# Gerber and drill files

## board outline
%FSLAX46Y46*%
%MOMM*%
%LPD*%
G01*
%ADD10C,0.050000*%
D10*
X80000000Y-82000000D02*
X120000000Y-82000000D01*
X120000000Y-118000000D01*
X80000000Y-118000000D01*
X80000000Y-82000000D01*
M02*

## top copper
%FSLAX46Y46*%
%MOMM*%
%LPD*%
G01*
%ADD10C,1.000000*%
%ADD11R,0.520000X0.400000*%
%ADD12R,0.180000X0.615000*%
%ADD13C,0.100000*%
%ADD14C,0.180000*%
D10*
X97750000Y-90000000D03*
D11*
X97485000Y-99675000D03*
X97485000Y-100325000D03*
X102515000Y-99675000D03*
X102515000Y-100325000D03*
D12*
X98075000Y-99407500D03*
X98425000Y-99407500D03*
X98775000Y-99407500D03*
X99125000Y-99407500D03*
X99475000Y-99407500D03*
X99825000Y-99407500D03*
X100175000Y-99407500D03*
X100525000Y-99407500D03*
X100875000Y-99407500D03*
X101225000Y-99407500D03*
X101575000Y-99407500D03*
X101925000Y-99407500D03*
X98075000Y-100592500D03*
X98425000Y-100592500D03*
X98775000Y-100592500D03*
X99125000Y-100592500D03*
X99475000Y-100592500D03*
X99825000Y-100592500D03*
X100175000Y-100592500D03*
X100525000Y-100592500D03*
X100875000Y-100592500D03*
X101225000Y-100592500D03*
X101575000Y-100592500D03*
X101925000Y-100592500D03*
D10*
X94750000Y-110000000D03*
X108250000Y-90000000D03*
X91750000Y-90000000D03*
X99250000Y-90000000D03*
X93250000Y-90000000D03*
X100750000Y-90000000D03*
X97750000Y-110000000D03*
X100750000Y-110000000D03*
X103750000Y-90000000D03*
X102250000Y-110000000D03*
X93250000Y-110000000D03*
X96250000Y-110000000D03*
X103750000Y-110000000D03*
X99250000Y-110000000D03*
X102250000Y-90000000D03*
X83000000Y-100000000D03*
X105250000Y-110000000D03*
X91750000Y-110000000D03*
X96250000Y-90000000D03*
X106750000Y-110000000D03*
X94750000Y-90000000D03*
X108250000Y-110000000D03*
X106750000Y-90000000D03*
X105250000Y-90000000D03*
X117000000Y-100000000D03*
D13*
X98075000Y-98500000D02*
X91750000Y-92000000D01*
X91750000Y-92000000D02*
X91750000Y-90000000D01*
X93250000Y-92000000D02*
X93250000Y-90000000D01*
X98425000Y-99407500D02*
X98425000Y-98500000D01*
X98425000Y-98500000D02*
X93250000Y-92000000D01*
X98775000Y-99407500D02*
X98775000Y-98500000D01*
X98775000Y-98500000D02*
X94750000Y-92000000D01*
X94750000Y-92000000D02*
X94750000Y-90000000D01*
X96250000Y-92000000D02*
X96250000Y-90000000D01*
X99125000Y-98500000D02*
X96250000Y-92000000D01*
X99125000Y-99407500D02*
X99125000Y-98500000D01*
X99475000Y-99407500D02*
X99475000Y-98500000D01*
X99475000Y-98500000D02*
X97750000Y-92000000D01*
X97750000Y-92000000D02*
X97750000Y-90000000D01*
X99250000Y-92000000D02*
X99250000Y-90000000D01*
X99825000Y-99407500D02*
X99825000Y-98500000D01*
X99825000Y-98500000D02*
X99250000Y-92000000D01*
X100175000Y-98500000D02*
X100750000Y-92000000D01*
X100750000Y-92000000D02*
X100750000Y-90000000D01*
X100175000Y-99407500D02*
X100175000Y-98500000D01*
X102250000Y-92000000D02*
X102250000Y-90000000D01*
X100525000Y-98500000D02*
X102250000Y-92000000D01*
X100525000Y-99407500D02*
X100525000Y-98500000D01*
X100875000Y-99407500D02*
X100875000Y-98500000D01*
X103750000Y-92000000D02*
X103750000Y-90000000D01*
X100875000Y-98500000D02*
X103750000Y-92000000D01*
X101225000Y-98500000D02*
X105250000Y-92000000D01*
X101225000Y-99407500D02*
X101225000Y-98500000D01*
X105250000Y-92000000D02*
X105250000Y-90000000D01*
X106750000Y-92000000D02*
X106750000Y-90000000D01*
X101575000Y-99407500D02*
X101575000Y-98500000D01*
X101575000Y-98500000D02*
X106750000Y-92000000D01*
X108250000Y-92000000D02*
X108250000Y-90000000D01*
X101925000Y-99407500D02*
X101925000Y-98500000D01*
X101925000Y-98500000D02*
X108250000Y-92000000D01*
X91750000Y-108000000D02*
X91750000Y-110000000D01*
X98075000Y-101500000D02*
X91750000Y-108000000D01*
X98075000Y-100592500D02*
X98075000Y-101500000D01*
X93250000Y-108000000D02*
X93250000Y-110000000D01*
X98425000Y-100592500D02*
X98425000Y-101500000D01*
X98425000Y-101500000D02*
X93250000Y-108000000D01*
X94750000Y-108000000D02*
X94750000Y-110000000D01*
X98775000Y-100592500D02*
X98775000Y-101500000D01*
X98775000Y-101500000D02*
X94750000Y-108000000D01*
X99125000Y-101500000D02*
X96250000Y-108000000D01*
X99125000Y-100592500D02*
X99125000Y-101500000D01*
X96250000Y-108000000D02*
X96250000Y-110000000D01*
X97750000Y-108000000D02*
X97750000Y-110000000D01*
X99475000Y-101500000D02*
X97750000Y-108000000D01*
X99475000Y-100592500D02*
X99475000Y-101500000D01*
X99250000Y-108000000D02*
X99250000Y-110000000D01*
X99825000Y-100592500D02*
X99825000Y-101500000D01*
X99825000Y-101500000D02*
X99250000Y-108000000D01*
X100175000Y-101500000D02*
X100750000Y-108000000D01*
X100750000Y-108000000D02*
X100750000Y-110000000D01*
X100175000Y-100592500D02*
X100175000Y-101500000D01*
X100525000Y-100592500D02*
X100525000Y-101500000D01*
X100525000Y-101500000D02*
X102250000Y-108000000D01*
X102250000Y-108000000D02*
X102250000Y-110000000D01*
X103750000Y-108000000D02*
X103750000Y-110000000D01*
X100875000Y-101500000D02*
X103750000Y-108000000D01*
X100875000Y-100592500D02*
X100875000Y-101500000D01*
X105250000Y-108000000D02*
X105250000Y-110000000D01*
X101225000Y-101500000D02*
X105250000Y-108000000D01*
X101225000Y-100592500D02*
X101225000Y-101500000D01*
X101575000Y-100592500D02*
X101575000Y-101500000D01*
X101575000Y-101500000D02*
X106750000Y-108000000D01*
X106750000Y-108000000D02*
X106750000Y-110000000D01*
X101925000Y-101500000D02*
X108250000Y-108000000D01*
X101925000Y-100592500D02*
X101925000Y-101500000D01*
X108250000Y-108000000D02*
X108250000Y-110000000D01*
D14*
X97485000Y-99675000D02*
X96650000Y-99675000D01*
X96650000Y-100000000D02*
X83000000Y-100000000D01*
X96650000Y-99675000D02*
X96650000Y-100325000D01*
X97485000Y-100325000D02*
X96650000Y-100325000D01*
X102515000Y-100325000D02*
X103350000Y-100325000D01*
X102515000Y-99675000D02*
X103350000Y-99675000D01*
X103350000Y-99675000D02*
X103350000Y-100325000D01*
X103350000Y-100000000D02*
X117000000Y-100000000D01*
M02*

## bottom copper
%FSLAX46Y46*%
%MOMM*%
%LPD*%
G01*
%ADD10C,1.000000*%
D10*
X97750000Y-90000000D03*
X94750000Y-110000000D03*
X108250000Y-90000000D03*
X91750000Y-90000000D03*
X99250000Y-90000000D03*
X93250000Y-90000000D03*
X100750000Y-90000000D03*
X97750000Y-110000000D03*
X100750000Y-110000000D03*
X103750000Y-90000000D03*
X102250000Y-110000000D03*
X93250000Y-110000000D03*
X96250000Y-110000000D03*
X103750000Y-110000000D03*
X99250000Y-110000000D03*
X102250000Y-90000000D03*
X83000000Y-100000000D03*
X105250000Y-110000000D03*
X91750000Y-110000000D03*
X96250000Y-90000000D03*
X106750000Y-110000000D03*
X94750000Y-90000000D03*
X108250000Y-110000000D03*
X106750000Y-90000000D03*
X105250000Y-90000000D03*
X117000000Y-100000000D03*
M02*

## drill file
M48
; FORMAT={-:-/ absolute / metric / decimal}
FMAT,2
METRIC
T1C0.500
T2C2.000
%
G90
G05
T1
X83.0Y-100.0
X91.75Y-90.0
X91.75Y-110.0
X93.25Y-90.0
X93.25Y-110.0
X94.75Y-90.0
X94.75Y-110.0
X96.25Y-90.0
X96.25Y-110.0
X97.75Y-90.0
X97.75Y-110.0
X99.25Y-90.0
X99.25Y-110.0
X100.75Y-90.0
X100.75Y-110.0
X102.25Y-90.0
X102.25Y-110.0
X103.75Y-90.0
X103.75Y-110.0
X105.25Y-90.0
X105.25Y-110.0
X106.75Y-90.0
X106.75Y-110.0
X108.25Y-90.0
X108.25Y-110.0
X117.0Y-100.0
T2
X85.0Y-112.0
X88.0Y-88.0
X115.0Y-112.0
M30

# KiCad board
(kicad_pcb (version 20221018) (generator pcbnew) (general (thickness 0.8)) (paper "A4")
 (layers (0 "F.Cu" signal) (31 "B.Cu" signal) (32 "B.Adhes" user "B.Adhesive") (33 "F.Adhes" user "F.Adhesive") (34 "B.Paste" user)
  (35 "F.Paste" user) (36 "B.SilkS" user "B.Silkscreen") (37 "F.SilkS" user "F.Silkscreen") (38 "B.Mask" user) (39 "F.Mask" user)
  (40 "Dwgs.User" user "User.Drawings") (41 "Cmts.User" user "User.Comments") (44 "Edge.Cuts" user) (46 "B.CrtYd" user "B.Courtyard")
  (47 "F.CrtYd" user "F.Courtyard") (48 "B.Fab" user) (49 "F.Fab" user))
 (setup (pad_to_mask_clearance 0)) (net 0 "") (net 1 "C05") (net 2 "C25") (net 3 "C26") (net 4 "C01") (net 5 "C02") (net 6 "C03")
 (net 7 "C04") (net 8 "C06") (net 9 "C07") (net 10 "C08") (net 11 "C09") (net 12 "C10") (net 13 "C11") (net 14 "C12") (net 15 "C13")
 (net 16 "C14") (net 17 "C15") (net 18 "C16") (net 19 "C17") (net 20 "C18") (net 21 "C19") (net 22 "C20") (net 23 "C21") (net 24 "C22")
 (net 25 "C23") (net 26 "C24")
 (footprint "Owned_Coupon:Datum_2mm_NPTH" (layer "F.Cu") (at 85 112)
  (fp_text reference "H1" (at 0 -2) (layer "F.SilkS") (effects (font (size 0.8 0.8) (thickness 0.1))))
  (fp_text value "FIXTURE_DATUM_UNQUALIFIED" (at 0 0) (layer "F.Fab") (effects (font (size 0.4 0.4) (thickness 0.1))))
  (pad "" np_thru_hole circle (at 0 0) (size 2 2) (drill 2) (layers "*.Cu" "*.Mask")))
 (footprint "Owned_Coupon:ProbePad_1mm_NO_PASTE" (layer "F.Cu") (at 97.75 90)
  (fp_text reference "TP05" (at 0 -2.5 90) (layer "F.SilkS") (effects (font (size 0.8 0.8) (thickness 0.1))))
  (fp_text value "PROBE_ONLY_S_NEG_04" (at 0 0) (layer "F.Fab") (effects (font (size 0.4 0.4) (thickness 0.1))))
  (pad "1" thru_hole circle (at 0 0) (size 1 1) (drill 0.5) (layers "*.Cu" "*.Mask") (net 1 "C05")))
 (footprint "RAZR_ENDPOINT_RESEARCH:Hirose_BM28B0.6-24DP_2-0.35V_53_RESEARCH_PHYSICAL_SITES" (layer "F.Cu") (at 100 100)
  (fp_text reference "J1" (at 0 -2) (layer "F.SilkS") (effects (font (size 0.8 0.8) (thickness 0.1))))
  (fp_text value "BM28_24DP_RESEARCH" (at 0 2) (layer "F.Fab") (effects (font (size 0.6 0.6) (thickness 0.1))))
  (pad "P_L" smd rect (at -2.515 -0.325) (size 0.52 0.4) (layers "F.Cu" "F.Mask") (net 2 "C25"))
  (pad "P_L" smd rect (at -2.515 0.325) (size 0.52 0.4) (layers "F.Cu" "F.Mask") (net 2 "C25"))
  (pad "P_R" smd rect (at 2.515 -0.325) (size 0.52 0.4) (layers "F.Cu" "F.Mask") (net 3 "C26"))
  (pad "P_R" smd rect (at 2.515 0.325) (size 0.52 0.4) (layers "F.Cu" "F.Mask") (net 3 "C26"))
  (pad "S_NEG_00" smd rect (at -1.925 -0.5925) (size 0.18 0.615) (layers "F.Cu" "F.Mask") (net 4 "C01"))
  (pad "S_NEG_01" smd rect (at -1.575 -0.5925) (size 0.18 0.615) (layers "F.Cu" "F.Mask") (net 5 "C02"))
  (pad "S_NEG_02" smd rect (at -1.225 -0.5925) (size 0.18 0.615) (layers "F.Cu" "F.Mask") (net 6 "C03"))
  (pad "S_NEG_03" smd rect (at -0.875 -0.5925) (size 0.18 0.615) (layers "F.Cu" "F.Mask") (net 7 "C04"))
  (pad "S_NEG_04" smd rect (at -0.525 -0.5925) (size 0.18 0.615) (layers "F.Cu" "F.Mask") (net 1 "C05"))
  (pad "S_NEG_05" smd rect (at -0.175 -0.5925) (size 0.18 0.615) (layers "F.Cu" "F.Mask") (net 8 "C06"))
  (pad "S_NEG_06" smd rect (at 0.175 -0.5925) (size 0.18 0.615) (layers "F.Cu" "F.Mask") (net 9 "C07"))
  (pad "S_NEG_07" smd rect (at 0.525 -0.5925) (size 0.18 0.615) (layers "F.Cu" "F.Mask") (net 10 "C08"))
  (pad "S_NEG_08" smd rect (at 0.875 -0.5925) (size 0.18 0.615) (layers "F.Cu" "F.Mask") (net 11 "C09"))
  (pad "S_NEG_09" smd rect (at 1.225 -0.5925) (size 0.18 0.615) (layers "F.Cu" "F.Mask") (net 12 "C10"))
  (pad "S_NEG_10" smd rect (at 1.575 -0.5925) (size 0.18 0.615) (layers "F.Cu" "F.Mask") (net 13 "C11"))
  (pad "S_NEG_11" smd rect (at 1.925 -0.5925) (size 0.18 0.615) (layers "F.Cu" "F.Mask") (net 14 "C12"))
  (pad "S_POS_00" smd rect (at -1.925 0.5925) (size 0.18 0.615) (layers "F.Cu" "F.Mask") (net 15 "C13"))
  (pad "S_POS_01" smd rect (at -1.575 0.5925) (size 0.18 0.615) (layers "F.Cu" "F.Mask") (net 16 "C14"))
  (pad "S_POS_02" smd rect (at -1.225 0.5925) (size 0.18 0.615) (layers "F.Cu" "F.Mask") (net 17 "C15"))
  (pad "S_POS_03" smd rect (at -0.875 0.5925) (size 0.18 0.615) (layers "F.Cu" "F.Mask") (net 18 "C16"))
  (pad "S_POS_04" smd rect (at -0.525 0.5925) (size 0.18 0.615) (layers "F.Cu" "F.Mask") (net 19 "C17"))
  (pad "S_POS_05" smd rect (at -0.175 0.5925) (size 0.18 0.615) (layers "F.Cu" "F.Mask") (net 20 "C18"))
  (pad "S_POS_06" smd rect (at 0.175 0.5925) (size 0.18 0.615) (layers "F.Cu" "F.Mask") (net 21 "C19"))
  (pad "S_POS_07" smd rect (at 0.525 0.5925) (size 0.18 0.615) (layers "F.Cu" "F.Mask") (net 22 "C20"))
  (pad "S_POS_08" smd rect (at 0.875 0.5925) (size 0.18 0.615) (layers "F.Cu" "F.Mask") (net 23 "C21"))
  (pad "S_POS_09" smd rect (at 1.225 0.5925) (size 0.18 0.615) (layers "F.Cu" "F.Mask") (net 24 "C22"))
  (pad "S_POS_10" smd rect (at 1.575 0.5925) (size 0.18 0.615) (layers "F.Cu" "F.Mask") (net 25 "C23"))
  (pad "S_POS_11" smd rect (at 1.925 0.5925) (size 0.18 0.615) (layers "F.Cu" "F.Mask") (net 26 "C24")))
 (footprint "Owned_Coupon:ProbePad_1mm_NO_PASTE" (layer "F.Cu") (at 94.75 110)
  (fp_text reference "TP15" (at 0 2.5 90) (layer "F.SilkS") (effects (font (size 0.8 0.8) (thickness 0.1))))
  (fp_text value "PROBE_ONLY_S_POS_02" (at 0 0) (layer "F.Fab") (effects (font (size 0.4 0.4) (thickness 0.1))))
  (pad "1" thru_hole circle (at 0 0) (size 1 1) (drill 0.5) (layers "*.Cu" "*.Mask") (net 17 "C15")))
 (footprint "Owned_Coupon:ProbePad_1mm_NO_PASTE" (layer "F.Cu") (at 108.25 90)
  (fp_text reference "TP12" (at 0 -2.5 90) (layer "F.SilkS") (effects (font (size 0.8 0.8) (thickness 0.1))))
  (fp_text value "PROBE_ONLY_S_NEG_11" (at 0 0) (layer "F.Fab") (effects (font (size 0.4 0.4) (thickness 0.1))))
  (pad "1" thru_hole circle (at 0 0) (size 1 1) (drill 0.5) (layers "*.Cu" "*.Mask") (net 14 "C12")))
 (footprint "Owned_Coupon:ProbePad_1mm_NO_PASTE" (layer "F.Cu") (at 91.75 90)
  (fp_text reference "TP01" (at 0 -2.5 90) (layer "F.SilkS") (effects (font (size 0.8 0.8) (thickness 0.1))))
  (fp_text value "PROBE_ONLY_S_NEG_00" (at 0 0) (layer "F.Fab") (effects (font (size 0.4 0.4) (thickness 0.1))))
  (pad "1" thru_hole circle (at 0 0) (size 1 1) (drill 0.5) (layers "*.Cu" "*.Mask") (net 4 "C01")))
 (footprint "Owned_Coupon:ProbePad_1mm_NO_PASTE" (layer "F.Cu") (at 99.25 90)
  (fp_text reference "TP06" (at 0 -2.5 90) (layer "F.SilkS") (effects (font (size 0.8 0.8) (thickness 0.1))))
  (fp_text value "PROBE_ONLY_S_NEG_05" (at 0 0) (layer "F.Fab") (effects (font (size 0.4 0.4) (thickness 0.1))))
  (pad "1" thru_hole circle (at 0 0) (size 1 1) (drill 0.5) (layers "*.Cu" "*.Mask") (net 8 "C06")))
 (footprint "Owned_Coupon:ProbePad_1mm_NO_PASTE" (layer "F.Cu") (at 93.25 90)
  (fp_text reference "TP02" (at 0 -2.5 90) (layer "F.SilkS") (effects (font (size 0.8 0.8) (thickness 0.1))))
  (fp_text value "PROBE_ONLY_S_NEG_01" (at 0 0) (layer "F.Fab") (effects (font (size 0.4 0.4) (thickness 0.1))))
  (pad "1" thru_hole circle (at 0 0) (size 1 1) (drill 0.5) (layers "*.Cu" "*.Mask") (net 5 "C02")))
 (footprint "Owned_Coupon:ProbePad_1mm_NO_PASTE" (layer "F.Cu") (at 100.75 90)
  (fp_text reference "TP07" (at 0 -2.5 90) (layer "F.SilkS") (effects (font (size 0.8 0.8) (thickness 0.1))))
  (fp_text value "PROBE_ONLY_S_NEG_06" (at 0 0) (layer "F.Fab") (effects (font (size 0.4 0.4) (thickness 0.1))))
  (pad "1" thru_hole circle (at 0 0) (size 1 1) (drill 0.5) (layers "*.Cu" "*.Mask") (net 9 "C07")))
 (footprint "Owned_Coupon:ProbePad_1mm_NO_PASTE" (layer "F.Cu") (at 97.75 110)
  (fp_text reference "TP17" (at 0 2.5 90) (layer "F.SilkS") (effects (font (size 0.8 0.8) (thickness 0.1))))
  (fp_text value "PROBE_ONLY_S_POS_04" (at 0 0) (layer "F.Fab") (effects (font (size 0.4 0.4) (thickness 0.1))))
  (pad "1" thru_hole circle (at 0 0) (size 1 1) (drill 0.5) (layers "*.Cu" "*.Mask") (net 19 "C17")))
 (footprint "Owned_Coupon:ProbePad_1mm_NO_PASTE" (layer "F.Cu") (at 100.75 110)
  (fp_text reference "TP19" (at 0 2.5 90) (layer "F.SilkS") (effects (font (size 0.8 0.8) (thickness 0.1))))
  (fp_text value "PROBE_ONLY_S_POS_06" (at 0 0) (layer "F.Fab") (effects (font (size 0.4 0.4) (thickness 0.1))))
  (pad "1" thru_hole circle (at 0 0) (size 1 1) (drill 0.5) (layers "*.Cu" "*.Mask") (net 21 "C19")))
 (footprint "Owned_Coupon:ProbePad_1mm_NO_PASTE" (layer "F.Cu") (at 103.75 90)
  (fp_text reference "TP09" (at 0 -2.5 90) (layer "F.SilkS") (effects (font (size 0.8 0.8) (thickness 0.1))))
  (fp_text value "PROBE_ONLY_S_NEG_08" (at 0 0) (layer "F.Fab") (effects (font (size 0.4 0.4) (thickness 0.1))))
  (pad "1" thru_hole circle (at 0 0) (size 1 1) (drill 0.5) (layers "*.Cu" "*.Mask") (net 11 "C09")))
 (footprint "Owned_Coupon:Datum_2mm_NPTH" (layer "F.Cu") (at 115 112)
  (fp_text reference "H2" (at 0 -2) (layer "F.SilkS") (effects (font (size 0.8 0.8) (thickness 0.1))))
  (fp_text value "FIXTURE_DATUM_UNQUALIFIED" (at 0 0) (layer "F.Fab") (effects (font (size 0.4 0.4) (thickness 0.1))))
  (pad "" np_thru_hole circle (at 0 0) (size 2 2) (drill 2) (layers "*.Cu" "*.Mask")))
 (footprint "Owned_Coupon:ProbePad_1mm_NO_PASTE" (layer "F.Cu") (at 102.25 110)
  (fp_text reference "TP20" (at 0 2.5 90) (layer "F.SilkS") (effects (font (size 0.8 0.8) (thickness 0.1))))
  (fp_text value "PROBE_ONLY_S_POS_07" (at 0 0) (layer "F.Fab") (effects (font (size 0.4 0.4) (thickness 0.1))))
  (pad "1" thru_hole circle (at 0 0) (size 1 1) (drill 0.5) (layers "*.Cu" "*.Mask") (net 22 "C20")))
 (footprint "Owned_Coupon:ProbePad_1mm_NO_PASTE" (layer "F.Cu") (at 93.25 110)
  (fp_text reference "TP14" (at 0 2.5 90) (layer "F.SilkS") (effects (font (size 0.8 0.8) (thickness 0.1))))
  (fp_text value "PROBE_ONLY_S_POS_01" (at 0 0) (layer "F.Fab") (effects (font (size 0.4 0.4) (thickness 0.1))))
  (pad "1" thru_hole circle (at 0 0) (size 1 1) (drill 0.5) (layers "*.Cu" "*.Mask") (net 16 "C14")))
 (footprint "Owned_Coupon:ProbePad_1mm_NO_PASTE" (layer "F.Cu") (at 96.25 110)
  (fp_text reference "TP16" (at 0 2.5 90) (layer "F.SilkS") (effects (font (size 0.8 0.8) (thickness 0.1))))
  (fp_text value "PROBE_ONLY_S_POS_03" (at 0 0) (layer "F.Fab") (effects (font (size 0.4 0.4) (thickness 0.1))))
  (pad "1" thru_hole circle (at 0 0) (size 1 1) (drill 0.5) (layers "*.Cu" "*.Mask") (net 18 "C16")))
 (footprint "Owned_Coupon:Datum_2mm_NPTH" (layer "F.Cu") (at 88 88)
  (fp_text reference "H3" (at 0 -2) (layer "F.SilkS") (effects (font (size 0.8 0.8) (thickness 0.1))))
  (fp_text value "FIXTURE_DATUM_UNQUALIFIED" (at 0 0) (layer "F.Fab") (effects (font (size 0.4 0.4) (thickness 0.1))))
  (pad "" np_thru_hole circle (at 0 0) (size 2 2) (drill 2) (layers "*.Cu" "*.Mask")))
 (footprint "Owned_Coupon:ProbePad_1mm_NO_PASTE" (layer "F.Cu") (at 103.75 110)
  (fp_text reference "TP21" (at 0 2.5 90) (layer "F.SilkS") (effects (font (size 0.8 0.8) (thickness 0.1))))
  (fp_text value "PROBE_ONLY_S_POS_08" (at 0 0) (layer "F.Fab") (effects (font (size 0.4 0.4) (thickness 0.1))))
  (pad "1" thru_hole circle (at 0 0) (size 1 1) (drill 0.5) (layers "*.Cu" "*.Mask") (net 23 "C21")))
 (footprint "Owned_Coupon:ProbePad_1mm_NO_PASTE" (layer "F.Cu") (at 99.25 110)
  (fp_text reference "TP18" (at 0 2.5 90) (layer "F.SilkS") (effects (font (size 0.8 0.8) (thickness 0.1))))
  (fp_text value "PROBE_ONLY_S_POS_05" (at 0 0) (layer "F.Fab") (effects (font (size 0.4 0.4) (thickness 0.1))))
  (pad "1" thru_hole circle (at 0 0) (size 1 1) (drill 0.5) (layers "*.Cu" "*.Mask") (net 20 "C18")))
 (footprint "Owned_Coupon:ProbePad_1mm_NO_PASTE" (layer "F.Cu") (at 102.25 90)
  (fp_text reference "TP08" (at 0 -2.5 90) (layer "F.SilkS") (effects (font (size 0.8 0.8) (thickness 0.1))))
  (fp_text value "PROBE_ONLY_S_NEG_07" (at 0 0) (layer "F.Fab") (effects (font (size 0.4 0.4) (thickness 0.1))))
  (pad "1" thru_hole circle (at 0 0) (size 1 1) (drill 0.5) (layers "*.Cu" "*.Mask") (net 10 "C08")))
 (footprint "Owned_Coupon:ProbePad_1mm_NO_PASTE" (layer "F.Cu") (at 83 100)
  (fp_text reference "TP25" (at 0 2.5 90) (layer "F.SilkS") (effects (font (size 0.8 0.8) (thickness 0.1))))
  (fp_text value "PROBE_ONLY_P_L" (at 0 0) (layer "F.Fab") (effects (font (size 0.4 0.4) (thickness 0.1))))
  (pad "1" thru_hole circle (at 0 0) (size 1 1) (drill 0.5) (layers "*.Cu" "*.Mask") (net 2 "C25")))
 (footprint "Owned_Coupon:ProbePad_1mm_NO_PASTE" (layer "F.Cu") (at 105.25 110)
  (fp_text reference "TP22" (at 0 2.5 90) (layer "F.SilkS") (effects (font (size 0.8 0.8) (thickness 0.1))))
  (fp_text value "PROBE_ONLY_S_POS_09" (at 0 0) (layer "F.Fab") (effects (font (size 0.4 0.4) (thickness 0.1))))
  (pad "1" thru_hole circle (at 0 0) (size 1 1) (drill 0.5) (layers "*.Cu" "*.Mask") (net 24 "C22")))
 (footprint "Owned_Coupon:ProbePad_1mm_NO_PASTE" (layer "F.Cu") (at 91.75 110)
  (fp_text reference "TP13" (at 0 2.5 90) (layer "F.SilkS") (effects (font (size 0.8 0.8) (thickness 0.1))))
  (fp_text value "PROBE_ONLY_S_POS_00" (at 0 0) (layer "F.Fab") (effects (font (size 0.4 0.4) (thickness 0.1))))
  (pad "1" thru_hole circle (at 0 0) (size 1 1) (drill 0.5) (layers "*.Cu" "*.Mask") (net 15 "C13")))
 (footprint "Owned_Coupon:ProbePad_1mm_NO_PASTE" (layer "F.Cu") (at 96.25 90)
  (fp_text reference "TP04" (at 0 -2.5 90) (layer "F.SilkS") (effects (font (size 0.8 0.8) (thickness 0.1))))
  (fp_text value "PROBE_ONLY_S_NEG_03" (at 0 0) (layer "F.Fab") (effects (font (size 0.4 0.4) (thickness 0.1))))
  (pad "1" thru_hole circle (at 0 0) (size 1 1) (drill 0.5) (layers "*.Cu" "*.Mask") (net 7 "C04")))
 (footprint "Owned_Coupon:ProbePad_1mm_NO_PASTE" (layer "F.Cu") (at 106.75 110)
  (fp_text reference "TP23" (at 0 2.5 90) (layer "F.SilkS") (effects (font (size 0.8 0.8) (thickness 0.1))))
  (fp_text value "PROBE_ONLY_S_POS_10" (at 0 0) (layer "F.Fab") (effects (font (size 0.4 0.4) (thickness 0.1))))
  (pad "1" thru_hole circle (at 0 0) (size 1 1) (drill 0.5) (layers "*.Cu" "*.Mask") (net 25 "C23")))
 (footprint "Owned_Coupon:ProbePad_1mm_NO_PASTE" (layer "F.Cu") (at 94.75 90)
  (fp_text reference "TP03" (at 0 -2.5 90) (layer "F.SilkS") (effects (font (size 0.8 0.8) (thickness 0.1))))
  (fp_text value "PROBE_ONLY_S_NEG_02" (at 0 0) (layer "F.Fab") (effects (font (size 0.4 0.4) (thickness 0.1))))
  (pad "1" thru_hole circle (at 0 0) (size 1 1) (drill 0.5) (layers "*.Cu" "*.Mask") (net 6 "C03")))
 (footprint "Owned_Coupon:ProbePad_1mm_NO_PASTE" (layer "F.Cu") (at 108.25 110)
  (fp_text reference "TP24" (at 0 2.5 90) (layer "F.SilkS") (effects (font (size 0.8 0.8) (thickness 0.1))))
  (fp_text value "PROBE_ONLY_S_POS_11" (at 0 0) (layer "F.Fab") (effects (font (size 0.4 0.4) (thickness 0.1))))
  (pad "1" thru_hole circle (at 0 0) (size 1 1) (drill 0.5) (layers "*.Cu" "*.Mask") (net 26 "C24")))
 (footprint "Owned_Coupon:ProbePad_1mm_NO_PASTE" (layer "F.Cu") (at 106.75 90)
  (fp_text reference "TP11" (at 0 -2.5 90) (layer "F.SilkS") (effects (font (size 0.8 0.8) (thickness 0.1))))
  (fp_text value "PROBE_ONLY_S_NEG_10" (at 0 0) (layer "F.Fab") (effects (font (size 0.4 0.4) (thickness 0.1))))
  (pad "1" thru_hole circle (at 0 0) (size 1 1) (drill 0.5) (layers "*.Cu" "*.Mask") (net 13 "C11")))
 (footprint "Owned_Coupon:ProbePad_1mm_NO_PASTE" (layer "F.Cu") (at 105.25 90)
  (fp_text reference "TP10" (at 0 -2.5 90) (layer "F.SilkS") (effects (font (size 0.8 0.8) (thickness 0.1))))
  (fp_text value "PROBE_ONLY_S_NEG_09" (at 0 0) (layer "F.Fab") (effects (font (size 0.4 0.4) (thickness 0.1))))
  (pad "1" thru_hole circle (at 0 0) (size 1 1) (drill 0.5) (layers "*.Cu" "*.Mask") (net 12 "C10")))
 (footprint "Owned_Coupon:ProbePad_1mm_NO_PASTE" (layer "F.Cu") (at 117 100)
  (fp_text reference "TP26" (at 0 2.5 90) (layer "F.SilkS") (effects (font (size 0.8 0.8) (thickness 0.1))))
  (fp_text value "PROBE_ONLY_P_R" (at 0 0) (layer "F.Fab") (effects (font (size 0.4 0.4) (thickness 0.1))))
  (pad "1" thru_hole circle (at 0 0) (size 1 1) (drill 0.5) (layers "*.Cu" "*.Mask") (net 3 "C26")))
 (gr_rect (start 80 82) (end 120 118) (stroke (width 0.05) (type default)) (fill none) (layer "Edge.Cuts"))
 (segment (start 98.075 98.5) (end 91.75 92) (width 0.1) (layer "F.Cu") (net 4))
 (segment (start 91.75 92) (end 91.75 90) (width 0.1) (layer "F.Cu") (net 4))
 (segment (start 93.25 92) (end 93.25 90) (width 0.1) (layer "F.Cu") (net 5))
 (segment (start 98.425 99.4075) (end 98.425 98.5) (width 0.1) (layer "F.Cu") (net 5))
 (segment (start 98.425 98.5) (end 93.25 92) (width 0.1) (layer "F.Cu") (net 5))
 (segment (start 98.775 99.4075) (end 98.775 98.5) (width 0.1) (layer "F.Cu") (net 6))
 (segment (start 98.775 98.5) (end 94.75 92) (width 0.1) (layer "F.Cu") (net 6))
 (segment (start 94.75 92) (end 94.75 90) (width 0.1) (layer "F.Cu") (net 6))
 (segment (start 96.25 92) (end 96.25 90) (width 0.1) (layer "F.Cu") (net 7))
 (segment (start 99.125 98.5) (end 96.25 92) (width 0.1) (layer "F.Cu") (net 7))
 (segment (start 99.125 99.4075) (end 99.125 98.5) (width 0.1) (layer "F.Cu") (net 7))
 (segment (start 99.475 99.4075) (end 99.475 98.5) (width 0.1) (layer "F.Cu") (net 1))
 (segment (start 99.475 98.5) (end 97.75 92) (width 0.1) (layer "F.Cu") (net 1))
 (segment (start 97.75 92) (end 97.75 90) (width 0.1) (layer "F.Cu") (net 1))
 (segment (start 99.25 92) (end 99.25 90) (width 0.1) (layer "F.Cu") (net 8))
 (segment (start 99.825 99.4075) (end 99.825 98.5) (width 0.1) (layer "F.Cu") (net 8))
 (segment (start 99.825 98.5) (end 99.25 92) (width 0.1) (layer "F.Cu") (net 8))
 (segment (start 100.175 98.5) (end 100.75 92) (width 0.1) (layer "F.Cu") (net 9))
 (segment (start 100.75 92) (end 100.75 90) (width 0.1) (layer "F.Cu") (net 9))
 (segment (start 100.175 99.4075) (end 100.175 98.5) (width 0.1) (layer "F.Cu") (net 9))
 (segment (start 102.25 92) (end 102.25 90) (width 0.1) (layer "F.Cu") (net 10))
 (segment (start 100.525 98.5) (end 102.25 92) (width 0.1) (layer "F.Cu") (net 10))
 (segment (start 100.525 99.4075) (end 100.525 98.5) (width 0.1) (layer "F.Cu") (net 10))
 (segment (start 100.875 99.4075) (end 100.875 98.5) (width 0.1) (layer "F.Cu") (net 11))
 (segment (start 103.75 92) (end 103.75 90) (width 0.1) (layer "F.Cu") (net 11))
 (segment (start 100.875 98.5) (end 103.75 92) (width 0.1) (layer "F.Cu") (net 11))
 (segment (start 101.225 98.5) (end 105.25 92) (width 0.1) (layer "F.Cu") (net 12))
 (segment (start 101.225 99.4075) (end 101.225 98.5) (width 0.1) (layer "F.Cu") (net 12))
 (segment (start 105.25 92) (end 105.25 90) (width 0.1) (layer "F.Cu") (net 12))
 (segment (start 106.75 92) (end 106.75 90) (width 0.1) (layer "F.Cu") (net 13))
 (segment (start 101.575 99.4075) (end 101.575 98.5) (width 0.1) (layer "F.Cu") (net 13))
 (segment (start 101.575 98.5) (end 106.75 92) (width 0.1) (layer "F.Cu") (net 13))
 (segment (start 108.25 92) (end 108.25 90) (width 0.1) (layer "F.Cu") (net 14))
 (segment (start 101.925 99.4075) (end 101.925 98.5) (width 0.1) (layer "F.Cu") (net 14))
 (segment (start 101.925 98.5) (end 108.25 92) (width 0.1) (layer "F.Cu") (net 14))
 (segment (start 91.75 108) (end 91.75 110) (width 0.1) (layer "F.Cu") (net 15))
 (segment (start 98.075 101.5) (end 91.75 108) (width 0.1) (layer "F.Cu") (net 15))
 (segment (start 98.075 100.5925) (end 98.075 101.5) (width 0.1) (layer "F.Cu") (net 15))
 (segment (start 93.25 108) (end 93.25 110) (width 0.1) (layer "F.Cu") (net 16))
 (segment (start 98.425 100.5925) (end 98.425 101.5) (width 0.1) (layer "F.Cu") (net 16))
 (segment (start 98.425 101.5) (end 93.25 108) (width 0.1) (layer "F.Cu") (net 16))
 (segment (start 94.75 108) (end 94.75 110) (width 0.1) (layer "F.Cu") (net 17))
 (segment (start 98.775 100.5925) (end 98.775 101.5) (width 0.1) (layer "F.Cu") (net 17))
 (segment (start 98.775 101.5) (end 94.75 108) (width 0.1) (layer "F.Cu") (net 17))
 (segment (start 99.125 101.5) (end 96.25 108) (width 0.1) (layer "F.Cu") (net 18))
 (segment (start 99.125 100.5925) (end 99.125 101.5) (width 0.1) (layer "F.Cu") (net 18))
 (segment (start 96.25 108) (end 96.25 110) (width 0.1) (layer "F.Cu") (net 18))
 (segment (start 97.75 108) (end 97.75 110) (width 0.1) (layer "F.Cu") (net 19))
 (segment (start 99.475 101.5) (end 97.75 108) (width 0.1) (layer "F.Cu") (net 19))
 (segment (start 99.475 100.5925) (end 99.475 101.5) (width 0.1) (layer "F.Cu") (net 19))
 (segment (start 99.25 108) (end 99.25 110) (width 0.1) (layer "F.Cu") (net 20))
 (segment (start 99.825 100.5925) (end 99.825 101.5) (width 0.1) (layer "F.Cu") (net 20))
 (segment (start 99.825 101.5) (end 99.25 108) (width 0.1) (layer "F.Cu") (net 20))
 (segment (start 100.175 101.5) (end 100.75 108) (width 0.1) (layer "F.Cu") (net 21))
 (segment (start 100.75 108) (end 100.75 110) (width 0.1) (layer "F.Cu") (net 21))
 (segment (start 100.175 100.5925) (end 100.175 101.5) (width 0.1) (layer "F.Cu") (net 21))
 (segment (start 100.525 100.5925) (end 100.525 101.5) (width 0.1) (layer "F.Cu") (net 22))
 (segment (start 100.525 101.5) (end 102.25 108) (width 0.1) (layer "F.Cu") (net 22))
 (segment (start 102.25 108) (end 102.25 110) (width 0.1) (layer "F.Cu") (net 22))
 (segment (start 103.75 108) (end 103.75 110) (width 0.1) (layer "F.Cu") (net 23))
 (segment (start 100.875 101.5) (end 103.75 108) (width 0.1) (layer "F.Cu") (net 23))
 (segment (start 100.875 100.5925) (end 100.875 101.5) (width 0.1) (layer "F.Cu") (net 23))
 (segment (start 105.25 108) (end 105.25 110) (width 0.1) (layer "F.Cu") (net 24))
 (segment (start 101.225 101.5) (end 105.25 108) (width 0.1) (layer "F.Cu") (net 24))
 (segment (start 101.225 100.5925) (end 101.225 101.5) (width 0.1) (layer "F.Cu") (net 24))
 (segment (start 101.575 100.5925) (end 101.575 101.5) (width 0.1) (layer "F.Cu") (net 25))
 (segment (start 101.575 101.5) (end 106.75 108) (width 0.1) (layer "F.Cu") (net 25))
 (segment (start 106.75 108) (end 106.75 110) (width 0.1) (layer "F.Cu") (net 25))
 (segment (start 101.925 101.5) (end 108.25 108) (width 0.1) (layer "F.Cu") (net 26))
 (segment (start 101.925 100.5925) (end 101.925 101.5) (width 0.1) (layer "F.Cu") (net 26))
 (segment (start 108.25 108) (end 108.25 110) (width 0.1) (layer "F.Cu") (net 26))
 (segment (start 97.485 99.675) (end 96.65 99.675) (width 0.18) (layer "F.Cu") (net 2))
 (segment (start 96.65 100) (end 83 100) (width 0.18) (layer "F.Cu") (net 2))
 (segment (start 96.65 99.675) (end 96.65 100.325) (width 0.18) (layer "F.Cu") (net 2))
 (segment (start 97.485 100.325) (end 96.65 100.325) (width 0.18) (layer "F.Cu") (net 2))
 (segment (start 102.515 100.325) (end 103.35 100.325) (width 0.18) (layer "F.Cu") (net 3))
 (segment (start 102.515 99.675) (end 103.35 99.675) (width 0.18) (layer "F.Cu") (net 3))
 (segment (start 103.35 99.675) (end 103.35 100.325) (width 0.18) (layer "F.Cu") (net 3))
 (segment (start 103.35 100) (end 117 100) (width 0.18) (layer "F.Cu") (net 3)))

